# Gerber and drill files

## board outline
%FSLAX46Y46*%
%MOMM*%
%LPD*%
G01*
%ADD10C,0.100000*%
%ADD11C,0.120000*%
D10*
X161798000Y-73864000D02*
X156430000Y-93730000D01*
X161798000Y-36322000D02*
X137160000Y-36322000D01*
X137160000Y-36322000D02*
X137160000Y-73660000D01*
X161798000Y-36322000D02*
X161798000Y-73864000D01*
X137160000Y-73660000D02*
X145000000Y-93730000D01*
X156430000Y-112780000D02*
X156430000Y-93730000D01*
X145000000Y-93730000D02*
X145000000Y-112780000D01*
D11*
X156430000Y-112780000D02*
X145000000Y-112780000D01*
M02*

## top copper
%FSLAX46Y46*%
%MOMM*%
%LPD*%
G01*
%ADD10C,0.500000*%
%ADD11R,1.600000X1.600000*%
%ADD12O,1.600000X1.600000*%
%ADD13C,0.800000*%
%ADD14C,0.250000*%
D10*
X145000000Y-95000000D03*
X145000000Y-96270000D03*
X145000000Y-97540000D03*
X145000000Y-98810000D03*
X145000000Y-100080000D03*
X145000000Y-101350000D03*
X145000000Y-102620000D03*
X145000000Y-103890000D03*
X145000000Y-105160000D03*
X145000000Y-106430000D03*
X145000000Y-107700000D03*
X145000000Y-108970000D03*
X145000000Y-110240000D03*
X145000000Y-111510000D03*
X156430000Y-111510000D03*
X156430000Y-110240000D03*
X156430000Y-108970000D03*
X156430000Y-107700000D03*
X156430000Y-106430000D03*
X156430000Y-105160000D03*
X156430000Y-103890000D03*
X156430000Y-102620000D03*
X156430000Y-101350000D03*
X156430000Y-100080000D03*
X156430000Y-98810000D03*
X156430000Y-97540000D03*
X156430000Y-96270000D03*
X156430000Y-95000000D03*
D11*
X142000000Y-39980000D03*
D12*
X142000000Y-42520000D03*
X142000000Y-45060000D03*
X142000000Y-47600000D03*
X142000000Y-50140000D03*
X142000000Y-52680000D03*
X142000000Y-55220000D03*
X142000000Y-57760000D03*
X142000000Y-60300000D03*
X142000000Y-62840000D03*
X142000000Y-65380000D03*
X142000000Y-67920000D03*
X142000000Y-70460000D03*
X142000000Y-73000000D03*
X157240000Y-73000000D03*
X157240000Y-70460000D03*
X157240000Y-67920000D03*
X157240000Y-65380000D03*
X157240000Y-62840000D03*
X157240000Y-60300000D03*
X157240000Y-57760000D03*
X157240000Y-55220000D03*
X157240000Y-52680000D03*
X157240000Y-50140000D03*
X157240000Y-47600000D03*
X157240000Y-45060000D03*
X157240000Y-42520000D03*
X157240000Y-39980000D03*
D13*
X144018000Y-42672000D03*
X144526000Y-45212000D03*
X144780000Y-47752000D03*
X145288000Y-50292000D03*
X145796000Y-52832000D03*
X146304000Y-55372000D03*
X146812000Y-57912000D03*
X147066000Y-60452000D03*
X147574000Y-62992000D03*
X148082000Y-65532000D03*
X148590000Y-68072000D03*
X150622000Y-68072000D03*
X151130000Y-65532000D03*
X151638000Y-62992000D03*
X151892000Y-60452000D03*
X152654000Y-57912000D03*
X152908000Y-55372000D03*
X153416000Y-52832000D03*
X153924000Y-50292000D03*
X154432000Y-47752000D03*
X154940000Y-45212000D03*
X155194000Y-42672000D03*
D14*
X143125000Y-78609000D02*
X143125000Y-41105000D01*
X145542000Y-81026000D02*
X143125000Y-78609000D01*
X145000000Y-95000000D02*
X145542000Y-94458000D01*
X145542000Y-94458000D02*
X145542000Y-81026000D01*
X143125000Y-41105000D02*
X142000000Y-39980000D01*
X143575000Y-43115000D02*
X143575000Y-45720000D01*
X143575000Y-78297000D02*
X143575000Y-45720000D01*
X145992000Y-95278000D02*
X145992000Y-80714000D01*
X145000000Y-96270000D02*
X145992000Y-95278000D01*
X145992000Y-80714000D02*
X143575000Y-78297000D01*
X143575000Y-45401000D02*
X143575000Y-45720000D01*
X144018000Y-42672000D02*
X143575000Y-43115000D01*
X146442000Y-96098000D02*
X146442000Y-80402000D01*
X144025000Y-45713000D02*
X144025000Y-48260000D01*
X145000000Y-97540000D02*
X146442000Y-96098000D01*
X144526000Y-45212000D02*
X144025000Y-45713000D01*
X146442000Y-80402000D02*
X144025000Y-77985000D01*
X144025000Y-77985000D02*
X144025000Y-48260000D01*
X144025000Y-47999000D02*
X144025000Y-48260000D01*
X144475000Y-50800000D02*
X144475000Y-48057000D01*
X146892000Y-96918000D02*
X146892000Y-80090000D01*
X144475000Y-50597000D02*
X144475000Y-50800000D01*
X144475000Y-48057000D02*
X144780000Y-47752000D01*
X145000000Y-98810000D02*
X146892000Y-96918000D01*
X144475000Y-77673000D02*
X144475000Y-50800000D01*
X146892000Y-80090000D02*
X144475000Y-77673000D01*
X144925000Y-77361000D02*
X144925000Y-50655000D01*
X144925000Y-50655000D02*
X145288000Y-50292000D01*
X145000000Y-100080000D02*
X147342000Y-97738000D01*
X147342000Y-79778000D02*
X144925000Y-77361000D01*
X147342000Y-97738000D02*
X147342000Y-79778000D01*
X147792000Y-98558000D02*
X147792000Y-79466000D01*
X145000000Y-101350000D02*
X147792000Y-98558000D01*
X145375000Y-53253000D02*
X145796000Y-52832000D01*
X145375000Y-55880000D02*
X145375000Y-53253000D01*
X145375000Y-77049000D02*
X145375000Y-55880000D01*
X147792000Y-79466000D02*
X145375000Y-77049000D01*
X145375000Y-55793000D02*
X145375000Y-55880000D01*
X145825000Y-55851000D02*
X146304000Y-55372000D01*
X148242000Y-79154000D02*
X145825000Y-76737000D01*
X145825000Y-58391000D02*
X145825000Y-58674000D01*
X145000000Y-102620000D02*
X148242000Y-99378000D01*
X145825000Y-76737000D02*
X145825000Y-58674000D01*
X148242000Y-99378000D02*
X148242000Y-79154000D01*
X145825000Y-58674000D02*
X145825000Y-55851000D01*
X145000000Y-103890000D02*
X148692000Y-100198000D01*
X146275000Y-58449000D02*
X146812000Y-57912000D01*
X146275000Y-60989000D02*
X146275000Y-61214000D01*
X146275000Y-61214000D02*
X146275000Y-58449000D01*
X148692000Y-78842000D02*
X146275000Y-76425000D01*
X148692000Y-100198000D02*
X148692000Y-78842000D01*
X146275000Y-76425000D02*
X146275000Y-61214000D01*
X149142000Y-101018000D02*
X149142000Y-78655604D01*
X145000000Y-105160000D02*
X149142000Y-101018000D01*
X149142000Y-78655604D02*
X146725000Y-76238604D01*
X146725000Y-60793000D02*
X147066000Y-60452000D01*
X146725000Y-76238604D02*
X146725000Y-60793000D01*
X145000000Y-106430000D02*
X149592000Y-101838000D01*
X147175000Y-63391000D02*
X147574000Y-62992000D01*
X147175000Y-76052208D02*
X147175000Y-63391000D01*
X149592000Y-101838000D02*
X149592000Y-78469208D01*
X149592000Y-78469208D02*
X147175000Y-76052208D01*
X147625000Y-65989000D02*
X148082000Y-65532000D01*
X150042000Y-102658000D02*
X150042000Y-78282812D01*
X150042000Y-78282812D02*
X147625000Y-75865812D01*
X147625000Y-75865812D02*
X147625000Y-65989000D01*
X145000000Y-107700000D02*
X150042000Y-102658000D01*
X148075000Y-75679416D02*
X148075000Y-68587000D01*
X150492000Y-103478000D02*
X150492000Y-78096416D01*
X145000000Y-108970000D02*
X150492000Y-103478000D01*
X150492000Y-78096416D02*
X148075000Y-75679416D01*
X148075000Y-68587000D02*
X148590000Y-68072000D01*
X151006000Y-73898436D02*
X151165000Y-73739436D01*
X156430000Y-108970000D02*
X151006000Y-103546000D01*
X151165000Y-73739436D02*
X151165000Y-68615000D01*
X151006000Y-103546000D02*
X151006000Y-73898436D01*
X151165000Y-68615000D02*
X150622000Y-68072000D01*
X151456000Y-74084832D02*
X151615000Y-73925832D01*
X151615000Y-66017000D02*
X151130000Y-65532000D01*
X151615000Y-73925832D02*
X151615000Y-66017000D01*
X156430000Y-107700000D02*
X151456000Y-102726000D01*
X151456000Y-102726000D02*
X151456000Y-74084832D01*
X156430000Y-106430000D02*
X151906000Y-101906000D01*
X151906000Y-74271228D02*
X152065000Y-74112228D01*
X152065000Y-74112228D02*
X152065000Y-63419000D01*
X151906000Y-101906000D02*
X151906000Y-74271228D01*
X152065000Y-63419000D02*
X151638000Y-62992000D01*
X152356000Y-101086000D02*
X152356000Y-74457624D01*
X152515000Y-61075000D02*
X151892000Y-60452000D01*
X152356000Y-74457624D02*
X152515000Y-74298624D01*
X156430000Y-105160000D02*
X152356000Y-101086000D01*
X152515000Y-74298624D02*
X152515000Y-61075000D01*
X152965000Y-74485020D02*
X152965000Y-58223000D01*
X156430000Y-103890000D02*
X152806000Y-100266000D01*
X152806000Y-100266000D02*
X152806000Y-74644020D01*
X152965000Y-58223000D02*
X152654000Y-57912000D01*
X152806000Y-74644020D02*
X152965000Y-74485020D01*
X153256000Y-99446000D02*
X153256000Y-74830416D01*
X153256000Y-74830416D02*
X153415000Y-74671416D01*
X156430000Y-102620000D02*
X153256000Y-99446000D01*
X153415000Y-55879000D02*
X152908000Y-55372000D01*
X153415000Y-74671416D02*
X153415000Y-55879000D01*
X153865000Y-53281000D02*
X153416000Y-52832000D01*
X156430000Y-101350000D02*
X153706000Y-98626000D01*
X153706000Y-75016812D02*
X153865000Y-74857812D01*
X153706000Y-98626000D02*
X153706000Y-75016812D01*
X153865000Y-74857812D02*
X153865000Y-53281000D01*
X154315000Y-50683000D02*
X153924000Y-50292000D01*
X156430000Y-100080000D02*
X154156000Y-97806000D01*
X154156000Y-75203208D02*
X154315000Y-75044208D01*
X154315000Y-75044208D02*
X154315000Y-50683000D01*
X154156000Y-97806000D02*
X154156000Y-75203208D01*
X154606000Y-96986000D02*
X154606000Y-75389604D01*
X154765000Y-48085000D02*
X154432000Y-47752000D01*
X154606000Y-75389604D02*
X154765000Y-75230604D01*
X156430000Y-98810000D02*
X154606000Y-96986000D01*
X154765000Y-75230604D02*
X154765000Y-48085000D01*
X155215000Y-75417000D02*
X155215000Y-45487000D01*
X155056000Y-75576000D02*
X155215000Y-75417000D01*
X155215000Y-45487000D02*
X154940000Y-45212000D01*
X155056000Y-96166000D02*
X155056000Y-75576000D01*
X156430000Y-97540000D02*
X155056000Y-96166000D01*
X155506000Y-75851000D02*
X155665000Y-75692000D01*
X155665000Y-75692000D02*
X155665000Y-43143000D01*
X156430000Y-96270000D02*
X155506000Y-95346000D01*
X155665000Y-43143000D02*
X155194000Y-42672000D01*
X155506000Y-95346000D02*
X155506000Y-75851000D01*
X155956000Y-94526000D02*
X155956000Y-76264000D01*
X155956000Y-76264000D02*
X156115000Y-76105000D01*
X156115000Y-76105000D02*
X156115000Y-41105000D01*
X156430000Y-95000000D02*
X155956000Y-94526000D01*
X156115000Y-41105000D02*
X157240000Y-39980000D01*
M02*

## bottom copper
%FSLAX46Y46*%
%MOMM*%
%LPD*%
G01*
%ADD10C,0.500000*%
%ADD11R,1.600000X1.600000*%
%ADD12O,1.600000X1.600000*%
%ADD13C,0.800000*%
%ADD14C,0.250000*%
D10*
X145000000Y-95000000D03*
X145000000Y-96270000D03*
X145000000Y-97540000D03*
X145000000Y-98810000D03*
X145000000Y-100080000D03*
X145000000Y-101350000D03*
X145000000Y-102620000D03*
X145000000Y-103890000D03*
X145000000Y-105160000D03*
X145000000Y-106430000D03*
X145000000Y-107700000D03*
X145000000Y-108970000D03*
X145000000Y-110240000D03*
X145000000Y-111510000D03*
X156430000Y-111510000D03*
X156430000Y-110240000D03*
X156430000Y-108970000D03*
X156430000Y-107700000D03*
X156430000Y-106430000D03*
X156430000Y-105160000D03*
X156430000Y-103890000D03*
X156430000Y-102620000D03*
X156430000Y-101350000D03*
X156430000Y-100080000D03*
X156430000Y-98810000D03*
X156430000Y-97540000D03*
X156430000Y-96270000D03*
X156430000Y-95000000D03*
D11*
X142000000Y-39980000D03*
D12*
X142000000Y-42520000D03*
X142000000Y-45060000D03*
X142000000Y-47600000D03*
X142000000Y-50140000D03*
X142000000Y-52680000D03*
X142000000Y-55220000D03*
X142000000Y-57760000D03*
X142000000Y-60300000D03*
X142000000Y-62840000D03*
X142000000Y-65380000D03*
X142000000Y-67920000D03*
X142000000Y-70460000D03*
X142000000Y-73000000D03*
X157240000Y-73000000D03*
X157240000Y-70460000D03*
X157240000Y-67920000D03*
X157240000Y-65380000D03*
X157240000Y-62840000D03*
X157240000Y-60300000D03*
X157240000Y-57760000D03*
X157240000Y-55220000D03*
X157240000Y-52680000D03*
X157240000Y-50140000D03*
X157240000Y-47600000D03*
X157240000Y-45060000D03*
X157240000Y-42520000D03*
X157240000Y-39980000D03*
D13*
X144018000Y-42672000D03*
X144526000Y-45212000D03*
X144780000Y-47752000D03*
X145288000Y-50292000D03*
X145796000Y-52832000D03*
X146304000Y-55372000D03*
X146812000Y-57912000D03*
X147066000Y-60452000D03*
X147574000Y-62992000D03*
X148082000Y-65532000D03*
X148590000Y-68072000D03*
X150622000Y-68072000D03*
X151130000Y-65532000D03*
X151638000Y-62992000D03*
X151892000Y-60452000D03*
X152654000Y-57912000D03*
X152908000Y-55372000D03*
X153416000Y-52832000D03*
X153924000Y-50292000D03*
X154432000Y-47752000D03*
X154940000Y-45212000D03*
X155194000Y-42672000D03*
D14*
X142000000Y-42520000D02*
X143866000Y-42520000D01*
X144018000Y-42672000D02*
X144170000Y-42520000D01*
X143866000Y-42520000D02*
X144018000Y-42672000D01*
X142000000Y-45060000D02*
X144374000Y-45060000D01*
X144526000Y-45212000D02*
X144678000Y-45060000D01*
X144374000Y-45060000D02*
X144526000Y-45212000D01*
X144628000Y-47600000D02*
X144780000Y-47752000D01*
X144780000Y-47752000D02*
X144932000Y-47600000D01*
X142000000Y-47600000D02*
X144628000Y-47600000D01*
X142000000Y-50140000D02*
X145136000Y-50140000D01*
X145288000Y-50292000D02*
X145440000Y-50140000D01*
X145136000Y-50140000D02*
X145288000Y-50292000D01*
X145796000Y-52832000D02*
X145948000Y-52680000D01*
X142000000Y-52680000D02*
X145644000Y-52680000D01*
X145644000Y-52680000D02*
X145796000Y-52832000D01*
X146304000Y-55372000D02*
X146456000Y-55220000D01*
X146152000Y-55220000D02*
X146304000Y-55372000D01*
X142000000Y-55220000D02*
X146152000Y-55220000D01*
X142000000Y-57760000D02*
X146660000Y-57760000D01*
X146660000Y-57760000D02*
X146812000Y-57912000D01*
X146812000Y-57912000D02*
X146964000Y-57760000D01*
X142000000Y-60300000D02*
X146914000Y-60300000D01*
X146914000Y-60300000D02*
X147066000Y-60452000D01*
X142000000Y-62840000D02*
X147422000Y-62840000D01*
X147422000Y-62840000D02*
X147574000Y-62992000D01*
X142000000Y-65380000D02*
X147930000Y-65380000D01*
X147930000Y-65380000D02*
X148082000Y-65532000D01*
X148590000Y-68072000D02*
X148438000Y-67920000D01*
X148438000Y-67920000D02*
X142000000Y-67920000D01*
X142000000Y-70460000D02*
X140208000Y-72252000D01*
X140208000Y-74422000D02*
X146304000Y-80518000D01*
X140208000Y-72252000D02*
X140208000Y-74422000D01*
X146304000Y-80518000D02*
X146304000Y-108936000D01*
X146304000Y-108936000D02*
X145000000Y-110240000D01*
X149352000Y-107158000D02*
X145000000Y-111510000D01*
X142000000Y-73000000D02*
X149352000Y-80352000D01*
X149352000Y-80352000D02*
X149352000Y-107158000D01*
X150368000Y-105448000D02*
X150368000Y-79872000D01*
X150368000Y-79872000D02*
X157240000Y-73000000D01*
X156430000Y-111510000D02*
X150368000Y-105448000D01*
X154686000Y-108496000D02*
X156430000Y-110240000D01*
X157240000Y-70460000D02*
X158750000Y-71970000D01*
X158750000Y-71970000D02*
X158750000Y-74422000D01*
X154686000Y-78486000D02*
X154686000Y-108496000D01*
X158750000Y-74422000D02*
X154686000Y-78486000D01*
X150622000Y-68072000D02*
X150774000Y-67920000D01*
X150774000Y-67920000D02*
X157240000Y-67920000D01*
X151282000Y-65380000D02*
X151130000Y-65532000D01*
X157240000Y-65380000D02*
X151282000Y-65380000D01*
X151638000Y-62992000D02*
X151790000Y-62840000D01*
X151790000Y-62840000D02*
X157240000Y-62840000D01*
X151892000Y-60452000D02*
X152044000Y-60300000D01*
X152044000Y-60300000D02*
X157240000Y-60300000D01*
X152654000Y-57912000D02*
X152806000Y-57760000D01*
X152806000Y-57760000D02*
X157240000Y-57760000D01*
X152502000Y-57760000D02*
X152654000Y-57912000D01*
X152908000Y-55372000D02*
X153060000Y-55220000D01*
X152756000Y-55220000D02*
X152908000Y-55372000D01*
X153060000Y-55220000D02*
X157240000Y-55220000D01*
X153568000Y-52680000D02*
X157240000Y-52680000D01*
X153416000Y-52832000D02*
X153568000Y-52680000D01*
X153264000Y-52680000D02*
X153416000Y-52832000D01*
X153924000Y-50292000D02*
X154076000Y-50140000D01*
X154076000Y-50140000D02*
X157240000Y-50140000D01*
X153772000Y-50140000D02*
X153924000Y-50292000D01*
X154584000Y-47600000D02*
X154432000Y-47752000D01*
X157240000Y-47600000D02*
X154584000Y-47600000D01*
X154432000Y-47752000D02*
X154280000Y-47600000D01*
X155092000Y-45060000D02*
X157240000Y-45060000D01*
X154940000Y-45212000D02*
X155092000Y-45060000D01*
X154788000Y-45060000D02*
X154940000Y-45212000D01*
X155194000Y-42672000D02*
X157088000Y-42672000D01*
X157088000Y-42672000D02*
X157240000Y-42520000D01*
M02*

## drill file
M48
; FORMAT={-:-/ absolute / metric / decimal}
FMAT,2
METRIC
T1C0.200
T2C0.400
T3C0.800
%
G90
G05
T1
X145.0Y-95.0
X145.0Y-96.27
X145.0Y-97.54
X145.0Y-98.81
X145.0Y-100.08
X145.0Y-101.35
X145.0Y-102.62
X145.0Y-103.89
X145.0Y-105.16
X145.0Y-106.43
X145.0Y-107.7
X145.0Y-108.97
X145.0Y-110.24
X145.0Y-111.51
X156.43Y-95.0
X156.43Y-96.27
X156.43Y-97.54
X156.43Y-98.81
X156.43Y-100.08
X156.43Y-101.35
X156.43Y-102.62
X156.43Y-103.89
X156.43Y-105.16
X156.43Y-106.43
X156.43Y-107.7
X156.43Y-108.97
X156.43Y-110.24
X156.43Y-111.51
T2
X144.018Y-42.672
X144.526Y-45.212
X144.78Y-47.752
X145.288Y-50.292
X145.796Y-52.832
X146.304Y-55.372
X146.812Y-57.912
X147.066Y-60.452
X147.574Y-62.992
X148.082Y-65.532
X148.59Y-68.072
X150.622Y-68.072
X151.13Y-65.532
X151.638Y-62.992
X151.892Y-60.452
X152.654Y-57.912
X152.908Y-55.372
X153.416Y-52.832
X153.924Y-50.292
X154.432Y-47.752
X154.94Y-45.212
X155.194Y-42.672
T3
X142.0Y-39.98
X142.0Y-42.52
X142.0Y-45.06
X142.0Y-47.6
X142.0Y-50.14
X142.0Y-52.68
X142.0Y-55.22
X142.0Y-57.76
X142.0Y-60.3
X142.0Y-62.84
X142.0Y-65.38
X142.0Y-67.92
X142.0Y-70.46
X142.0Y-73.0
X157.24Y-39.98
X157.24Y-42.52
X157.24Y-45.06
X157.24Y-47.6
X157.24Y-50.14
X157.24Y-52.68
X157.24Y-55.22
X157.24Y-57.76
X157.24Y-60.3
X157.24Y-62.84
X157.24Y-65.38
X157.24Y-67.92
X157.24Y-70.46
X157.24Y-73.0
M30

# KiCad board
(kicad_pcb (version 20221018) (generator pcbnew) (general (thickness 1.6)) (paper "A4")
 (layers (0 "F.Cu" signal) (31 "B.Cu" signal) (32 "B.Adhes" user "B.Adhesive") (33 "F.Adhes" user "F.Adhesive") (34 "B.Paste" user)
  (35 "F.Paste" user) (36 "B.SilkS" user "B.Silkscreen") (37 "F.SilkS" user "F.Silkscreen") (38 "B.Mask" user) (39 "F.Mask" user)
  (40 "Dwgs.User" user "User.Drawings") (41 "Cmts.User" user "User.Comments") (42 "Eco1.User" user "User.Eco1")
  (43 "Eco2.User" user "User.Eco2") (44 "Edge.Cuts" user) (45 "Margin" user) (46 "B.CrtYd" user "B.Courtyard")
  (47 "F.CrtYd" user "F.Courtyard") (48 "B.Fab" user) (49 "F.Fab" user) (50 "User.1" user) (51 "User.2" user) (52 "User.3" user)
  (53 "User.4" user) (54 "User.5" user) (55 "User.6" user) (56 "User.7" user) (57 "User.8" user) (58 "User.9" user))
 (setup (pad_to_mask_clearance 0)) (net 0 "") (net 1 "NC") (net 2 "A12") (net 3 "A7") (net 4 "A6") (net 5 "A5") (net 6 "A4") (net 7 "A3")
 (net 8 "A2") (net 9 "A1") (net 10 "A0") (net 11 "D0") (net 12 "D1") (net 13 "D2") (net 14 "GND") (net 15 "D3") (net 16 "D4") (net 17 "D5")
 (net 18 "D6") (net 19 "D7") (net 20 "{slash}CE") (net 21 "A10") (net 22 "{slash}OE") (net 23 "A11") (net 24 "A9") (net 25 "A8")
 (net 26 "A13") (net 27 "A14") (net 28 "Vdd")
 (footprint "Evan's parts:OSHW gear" (layer "F.Cu") (at 149.86 45.212)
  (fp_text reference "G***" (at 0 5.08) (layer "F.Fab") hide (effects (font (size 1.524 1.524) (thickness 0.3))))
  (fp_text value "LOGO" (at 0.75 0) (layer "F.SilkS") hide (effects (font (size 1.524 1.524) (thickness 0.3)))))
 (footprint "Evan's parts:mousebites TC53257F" (layer "F.Cu") (at 145 95)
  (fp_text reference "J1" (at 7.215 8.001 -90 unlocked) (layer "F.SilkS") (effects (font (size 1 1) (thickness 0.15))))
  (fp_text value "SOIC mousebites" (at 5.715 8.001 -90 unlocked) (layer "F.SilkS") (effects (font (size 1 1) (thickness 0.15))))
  (fp_line (start 11.43 17.78) (end 0 17.78) (stroke (width 0.12) (type default)) (layer "Edge.Cuts"))
  (pad "1" thru_hole circle (at 0 0) (size 0.5 0.5) (drill 0.2) (layers "*.Cu" "*.Mask") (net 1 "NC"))
  (pad "2" thru_hole circle (at 0 1.27) (size 0.5 0.5) (drill 0.2) (layers "*.Cu" "*.Mask") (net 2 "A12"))
  (pad "3" thru_hole circle (at 0 2.54) (size 0.5 0.5) (drill 0.2) (layers "*.Cu" "*.Mask") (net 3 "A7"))
  (pad "4" thru_hole circle (at 0 3.81) (size 0.5 0.5) (drill 0.2) (layers "*.Cu" "*.Mask") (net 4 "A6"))
  (pad "5" thru_hole circle (at 0 5.08) (size 0.5 0.5) (drill 0.2) (layers "*.Cu" "*.Mask") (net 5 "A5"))
  (pad "6" thru_hole circle (at 0 6.35) (size 0.5 0.5) (drill 0.2) (layers "*.Cu" "*.Mask") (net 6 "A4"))
  (pad "7" thru_hole circle (at 0 7.62) (size 0.5 0.5) (drill 0.2) (layers "*.Cu" "*.Mask") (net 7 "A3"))
  (pad "8" thru_hole circle (at 0 8.89) (size 0.5 0.5) (drill 0.2) (layers "*.Cu" "*.Mask") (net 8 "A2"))
  (pad "9" thru_hole circle (at 0 10.16) (size 0.5 0.5) (drill 0.2) (layers "*.Cu" "*.Mask") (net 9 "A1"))
  (pad "10" thru_hole circle (at 0 11.43) (size 0.5 0.5) (drill 0.2) (layers "*.Cu" "*.Mask") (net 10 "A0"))
  (pad "11" thru_hole circle (at 0 12.7) (size 0.5 0.5) (drill 0.2) (layers "*.Cu" "*.Mask") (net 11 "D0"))
  (pad "12" thru_hole circle (at 0 13.97) (size 0.5 0.5) (drill 0.2) (layers "*.Cu" "*.Mask") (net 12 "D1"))
  (pad "13" thru_hole circle (at 0 15.24) (size 0.5 0.5) (drill 0.2) (layers "*.Cu" "*.Mask") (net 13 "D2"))
  (pad "14" thru_hole circle (at 0 16.51) (size 0.5 0.5) (drill 0.2) (layers "*.Cu" "*.Mask") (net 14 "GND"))
  (pad "15" thru_hole circle (at 11.43 16.51) (size 0.5 0.5) (drill 0.2) (layers "*.Cu" "*.Mask") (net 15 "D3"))
  (pad "16" thru_hole circle (at 11.43 15.24) (size 0.5 0.5) (drill 0.2) (layers "*.Cu" "*.Mask") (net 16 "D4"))
  (pad "17" thru_hole circle (at 11.43 13.97) (size 0.5 0.5) (drill 0.2) (layers "*.Cu" "*.Mask") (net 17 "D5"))
  (pad "18" thru_hole circle (at 11.43 12.7) (size 0.5 0.5) (drill 0.2) (layers "*.Cu" "*.Mask") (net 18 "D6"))
  (pad "19" thru_hole circle (at 11.43 11.43) (size 0.5 0.5) (drill 0.2) (layers "*.Cu" "*.Mask") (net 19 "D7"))
  (pad "20" thru_hole circle (at 11.43 10.16) (size 0.5 0.5) (drill 0.2) (layers "*.Cu" "*.Mask") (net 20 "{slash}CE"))
  (pad "21" thru_hole circle (at 11.43 8.89) (size 0.5 0.5) (drill 0.2) (layers "*.Cu" "*.Mask") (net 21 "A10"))
  (pad "22" thru_hole circle (at 11.43 7.62) (size 0.5 0.5) (drill 0.2) (layers "*.Cu" "*.Mask") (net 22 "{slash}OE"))
  (pad "23" thru_hole circle (at 11.43 6.35) (size 0.5 0.5) (drill 0.2) (layers "*.Cu" "*.Mask") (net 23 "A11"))
  (pad "24" thru_hole circle (at 11.43 5.08) (size 0.5 0.5) (drill 0.2) (layers "*.Cu" "*.Mask") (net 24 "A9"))
  (pad "25" thru_hole circle (at 11.43 3.81) (size 0.5 0.5) (drill 0.2) (layers "*.Cu" "*.Mask") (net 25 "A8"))
  (pad "26" thru_hole circle (at 11.43 2.54) (size 0.5 0.5) (drill 0.2) (layers "*.Cu" "*.Mask") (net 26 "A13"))
  (pad "27" thru_hole circle (at 11.43 1.27) (size 0.5 0.5) (drill 0.2) (layers "*.Cu" "*.Mask") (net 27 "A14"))
  (pad "28" thru_hole circle (at 11.43 0) (size 0.5 0.5) (drill 0.2) (layers "*.Cu" "*.Mask") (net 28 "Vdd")))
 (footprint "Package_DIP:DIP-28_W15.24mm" (layer "F.Cu") (at 142 39.98)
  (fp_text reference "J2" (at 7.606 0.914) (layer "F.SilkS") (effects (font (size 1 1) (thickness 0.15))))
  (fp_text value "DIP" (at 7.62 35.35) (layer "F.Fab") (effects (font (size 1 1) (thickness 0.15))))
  (pad "1" thru_hole rect (at 0 0) (size 1.6 1.6) (drill 0.8) (layers "*.Cu" "*.Mask") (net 1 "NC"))
  (pad "2" thru_hole oval (at 0 2.54) (size 1.6 1.6) (drill 0.8) (layers "*.Cu" "*.Mask") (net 2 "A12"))
  (pad "3" thru_hole oval (at 0 5.08) (size 1.6 1.6) (drill 0.8) (layers "*.Cu" "*.Mask") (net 3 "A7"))
  (pad "4" thru_hole oval (at 0 7.62) (size 1.6 1.6) (drill 0.8) (layers "*.Cu" "*.Mask") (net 4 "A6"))
  (pad "5" thru_hole oval (at 0 10.16) (size 1.6 1.6) (drill 0.8) (layers "*.Cu" "*.Mask") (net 5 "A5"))
  (pad "6" thru_hole oval (at 0 12.7) (size 1.6 1.6) (drill 0.8) (layers "*.Cu" "*.Mask") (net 6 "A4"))
  (pad "7" thru_hole oval (at 0 15.24) (size 1.6 1.6) (drill 0.8) (layers "*.Cu" "*.Mask") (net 7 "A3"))
  (pad "8" thru_hole oval (at 0 17.78) (size 1.6 1.6) (drill 0.8) (layers "*.Cu" "*.Mask") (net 8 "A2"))
  (pad "9" thru_hole oval (at 0 20.32) (size 1.6 1.6) (drill 0.8) (layers "*.Cu" "*.Mask") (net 9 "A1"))
  (pad "10" thru_hole oval (at 0 22.86) (size 1.6 1.6) (drill 0.8) (layers "*.Cu" "*.Mask") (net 10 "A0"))
  (pad "11" thru_hole oval (at 0 25.4) (size 1.6 1.6) (drill 0.8) (layers "*.Cu" "*.Mask") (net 11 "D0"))
  (pad "12" thru_hole oval (at 0 27.94) (size 1.6 1.6) (drill 0.8) (layers "*.Cu" "*.Mask") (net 12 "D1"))
  (pad "13" thru_hole oval (at 0 30.48) (size 1.6 1.6) (drill 0.8) (layers "*.Cu" "*.Mask") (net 13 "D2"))
  (pad "14" thru_hole oval (at 0 33.02) (size 1.6 1.6) (drill 0.8) (layers "*.Cu" "*.Mask") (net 14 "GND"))
  (pad "15" thru_hole oval (at 15.24 33.02) (size 1.6 1.6) (drill 0.8) (layers "*.Cu" "*.Mask") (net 15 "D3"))
  (pad "16" thru_hole oval (at 15.24 30.48) (size 1.6 1.6) (drill 0.8) (layers "*.Cu" "*.Mask") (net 16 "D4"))
  (pad "17" thru_hole oval (at 15.24 27.94) (size 1.6 1.6) (drill 0.8) (layers "*.Cu" "*.Mask") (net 17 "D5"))
  (pad "18" thru_hole oval (at 15.24 25.4) (size 1.6 1.6) (drill 0.8) (layers "*.Cu" "*.Mask") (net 18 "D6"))
  (pad "19" thru_hole oval (at 15.24 22.86) (size 1.6 1.6) (drill 0.8) (layers "*.Cu" "*.Mask") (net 19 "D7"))
  (pad "20" thru_hole oval (at 15.24 20.32) (size 1.6 1.6) (drill 0.8) (layers "*.Cu" "*.Mask") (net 20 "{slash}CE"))
  (pad "21" thru_hole oval (at 15.24 17.78) (size 1.6 1.6) (drill 0.8) (layers "*.Cu" "*.Mask") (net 21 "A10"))
  (pad "22" thru_hole oval (at 15.24 15.24) (size 1.6 1.6) (drill 0.8) (layers "*.Cu" "*.Mask") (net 22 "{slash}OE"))
  (pad "23" thru_hole oval (at 15.24 12.7) (size 1.6 1.6) (drill 0.8) (layers "*.Cu" "*.Mask") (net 23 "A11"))
  (pad "24" thru_hole oval (at 15.24 10.16) (size 1.6 1.6) (drill 0.8) (layers "*.Cu" "*.Mask") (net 24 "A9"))
  (pad "25" thru_hole oval (at 15.24 7.62) (size 1.6 1.6) (drill 0.8) (layers "*.Cu" "*.Mask") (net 25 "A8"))
  (pad "26" thru_hole oval (at 15.24 5.08) (size 1.6 1.6) (drill 0.8) (layers "*.Cu" "*.Mask") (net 26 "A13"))
  (pad "27" thru_hole oval (at 15.24 2.54) (size 1.6 1.6) (drill 0.8) (layers "*.Cu" "*.Mask") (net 27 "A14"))
  (pad "28" thru_hole oval (at 15.24 0) (size 1.6 1.6) (drill 0.8) (layers "*.Cu" "*.Mask") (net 28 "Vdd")))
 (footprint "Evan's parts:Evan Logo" (layer "B.Cu") (at 149.86 41.402 -90)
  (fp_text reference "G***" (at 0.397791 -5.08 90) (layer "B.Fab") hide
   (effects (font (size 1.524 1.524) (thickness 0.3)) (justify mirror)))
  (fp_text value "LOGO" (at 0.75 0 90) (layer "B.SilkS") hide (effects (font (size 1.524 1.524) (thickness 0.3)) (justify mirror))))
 (gr_line (start 161.798 73.864) (end 156.43 93.73) (stroke (width 0.1) (type default)) (layer "Edge.Cuts"))
 (gr_line (start 161.798 36.322) (end 137.16 36.322) (stroke (width 0.1) (type default)) (layer "Edge.Cuts"))
 (gr_line (start 137.16 36.322) (end 137.16 73.66) (stroke (width 0.1) (type default)) (layer "Edge.Cuts"))
 (gr_line (start 161.798 36.322) (end 161.798 73.864) (stroke (width 0.1) (type default)) (layer "Edge.Cuts"))
 (gr_line (start 137.16 73.66) (end 145 93.73) (stroke (width 0.1) (type default)) (layer "Edge.Cuts"))
 (gr_line (start 156.43 112.78) (end 156.43 93.73) (stroke (width 0.1) (type default)) (layer "Edge.Cuts"))
 (gr_line (start 145 93.73) (end 145 112.78) (stroke (width 0.1) (type default)) (layer "Edge.Cuts"))
 (segment (start 143.125 78.609) (end 143.125 41.105) (width 0.25) (layer "F.Cu") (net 1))
 (segment (start 145.542 81.026) (end 143.125 78.609) (width 0.25) (layer "F.Cu") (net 1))
 (segment (start 145 95) (end 145.542 94.458) (width 0.25) (layer "F.Cu") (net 1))
 (segment (start 145.542 94.458) (end 145.542 81.026) (width 0.25) (layer "F.Cu") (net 1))
 (segment (start 143.125 41.105) (end 142 39.98) (width 0.25) (layer "F.Cu") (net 1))
 (segment (start 143.575 43.115) (end 143.575 45.72) (width 0.25) (layer "F.Cu") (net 2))
 (segment (start 143.575 78.297) (end 143.575 45.72) (width 0.25) (layer "F.Cu") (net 2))
 (segment (start 145.992 95.278) (end 145.992 80.714) (width 0.25) (layer "F.Cu") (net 2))
 (segment (start 145 96.27) (end 145.992 95.278) (width 0.25) (layer "F.Cu") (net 2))
 (segment (start 145.992 80.714) (end 143.575 78.297) (width 0.25) (layer "F.Cu") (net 2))
 (segment (start 143.575 45.401) (end 143.575 45.72) (width 0.25) (layer "F.Cu") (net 2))
 (segment (start 144.018 42.672) (end 143.575 43.115) (width 0.25) (layer "F.Cu") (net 2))
 (via (at 144.018 42.672) (size 0.8) (drill 0.4) (layers "F.Cu" "B.Cu") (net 2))
 (segment (start 142 42.52) (end 143.866 42.52) (width 0.25) (layer "B.Cu") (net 2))
 (segment (start 144.018 42.672) (end 144.17 42.52) (width 0.25) (layer "B.Cu") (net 2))
 (segment (start 143.866 42.52) (end 144.018 42.672) (width 0.25) (layer "B.Cu") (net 2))
 (segment (start 146.442 96.098) (end 146.442 80.402) (width 0.25) (layer "F.Cu") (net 3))
 (segment (start 144.025 45.713) (end 144.025 48.26) (width 0.25) (layer "F.Cu") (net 3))
 (segment (start 145 97.54) (end 146.442 96.098) (width 0.25) (layer "F.Cu") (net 3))
 (segment (start 144.526 45.212) (end 144.025 45.713) (width 0.25) (layer "F.Cu") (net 3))
 (segment (start 146.442 80.402) (end 144.025 77.985) (width 0.25) (layer "F.Cu") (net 3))
 (segment (start 144.025 77.985) (end 144.025 48.26) (width 0.25) (layer "F.Cu") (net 3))
 (segment (start 144.025 47.999) (end 144.025 48.26) (width 0.25) (layer "F.Cu") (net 3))
 (via (at 144.526 45.212) (size 0.8) (drill 0.4) (layers "F.Cu" "B.Cu") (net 3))
 (segment (start 142 45.06) (end 144.374 45.06) (width 0.25) (layer "B.Cu") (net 3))
 (segment (start 144.526 45.212) (end 144.678 45.06) (width 0.25) (layer "B.Cu") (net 3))
 (segment (start 144.374 45.06) (end 144.526 45.212) (width 0.25) (layer "B.Cu") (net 3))
 (segment (start 144.475 50.8) (end 144.475 48.057) (width 0.25) (layer "F.Cu") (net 4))
 (segment (start 146.892 96.918) (end 146.892 80.09) (width 0.25) (layer "F.Cu") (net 4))
 (segment (start 144.475 50.597) (end 144.475 50.8) (width 0.25) (layer "F.Cu") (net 4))
 (segment (start 144.475 48.057) (end 144.78 47.752) (width 0.25) (layer "F.Cu") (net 4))
 (segment (start 145 98.81) (end 146.892 96.918) (width 0.25) (layer "F.Cu") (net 4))
 (segment (start 144.475 77.673) (end 144.475 50.8) (width 0.25) (layer "F.Cu") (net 4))
 (segment (start 146.892 80.09) (end 144.475 77.673) (width 0.25) (layer "F.Cu") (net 4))
 (via (at 144.78 47.752) (size 0.8) (drill 0.4) (layers "F.Cu" "B.Cu") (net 4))
 (segment (start 144.628 47.6) (end 144.78 47.752) (width 0.25) (layer "B.Cu") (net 4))
 (segment (start 144.78 47.752) (end 144.932 47.6) (width 0.25) (layer "B.Cu") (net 4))
 (segment (start 142 47.6) (end 144.628 47.6) (width 0.25) (layer "B.Cu") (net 4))
 (segment (start 144.925 77.361) (end 144.925 50.655) (width 0.25) (layer "F.Cu") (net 5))
 (segment (start 144.925 50.655) (end 145.288 50.292) (width 0.25) (layer "F.Cu") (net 5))
 (segment (start 145 100.08) (end 147.342 97.738) (width 0.25) (layer "F.Cu") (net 5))
 (segment (start 147.342 79.778) (end 144.925 77.361) (width 0.25) (layer "F.Cu") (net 5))
 (segment (start 147.342 97.738) (end 147.342 79.778) (width 0.25) (layer "F.Cu") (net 5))
 (via (at 145.288 50.292) (size 0.8) (drill 0.4) (layers "F.Cu" "B.Cu") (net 5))
 (segment (start 142 50.14) (end 145.136 50.14) (width 0.25) (layer "B.Cu") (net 5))
 (segment (start 145.288 50.292) (end 145.44 50.14) (width 0.25) (layer "B.Cu") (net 5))
 (segment (start 145.136 50.14) (end 145.288 50.292) (width 0.25) (layer "B.Cu") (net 5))
 (segment (start 147.792 98.558) (end 147.792 79.466) (width 0.25) (layer "F.Cu") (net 6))
 (segment (start 145 101.35) (end 147.792 98.558) (width 0.25) (layer "F.Cu") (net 6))
 (segment (start 145.375 53.253) (end 145.796 52.832) (width 0.25) (layer "F.Cu") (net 6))
 (segment (start 145.375 55.88) (end 145.375 53.253) (width 0.25) (layer "F.Cu") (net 6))
 (segment (start 145.375 77.049) (end 145.375 55.88) (width 0.25) (layer "F.Cu") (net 6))
 (segment (start 147.792 79.466) (end 145.375 77.049) (width 0.25) (layer "F.Cu") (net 6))
 (segment (start 145.375 55.793) (end 145.375 55.88) (width 0.25) (layer "F.Cu") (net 6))
 (via (at 145.796 52.832) (size 0.8) (drill 0.4) (layers "F.Cu" "B.Cu") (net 6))
 (segment (start 145.796 52.832) (end 145.948 52.68) (width 0.25) (layer "B.Cu") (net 6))
 (segment (start 142 52.68) (end 145.644 52.68) (width 0.25) (layer "B.Cu") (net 6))
 (segment (start 145.644 52.68) (end 145.796 52.832) (width 0.25) (layer "B.Cu") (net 6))
 (segment (start 145.825 55.851) (end 146.304 55.372) (width 0.25) (layer "F.Cu") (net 7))
 (segment (start 148.242 79.154) (end 145.825 76.737) (width 0.25) (layer "F.Cu") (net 7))
 (segment (start 145.825 58.391) (end 145.825 58.674) (width 0.25) (layer "F.Cu") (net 7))
 (segment (start 145 102.62) (end 148.242 99.378) (width 0.25) (layer "F.Cu") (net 7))
 (segment (start 145.825 76.737) (end 145.825 58.674) (width 0.25) (layer "F.Cu") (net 7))
 (segment (start 148.242 99.378) (end 148.242 79.154) (width 0.25) (layer "F.Cu") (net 7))
 (segment (start 145.825 58.674) (end 145.825 55.851) (width 0.25) (layer "F.Cu") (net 7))
 (via (at 146.304 55.372) (size 0.8) (drill 0.4) (layers "F.Cu" "B.Cu") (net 7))
 (segment (start 146.304 55.372) (end 146.456 55.22) (width 0.25) (layer "B.Cu") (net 7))
 (segment (start 146.152 55.22) (end 146.304 55.372) (width 0.25) (layer "B.Cu") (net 7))
 (segment (start 142 55.22) (end 146.152 55.22) (width 0.25) (layer "B.Cu") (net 7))
 (segment (start 145 103.89) (end 148.692 100.198) (width 0.25) (layer "F.Cu") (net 8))
 (segment (start 146.275 58.449) (end 146.812 57.912) (width 0.25) (layer "F.Cu") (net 8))
 (segment (start 146.275 60.989) (end 146.275 61.214) (width 0.25) (layer "F.Cu") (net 8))
 (segment (start 146.275 61.214) (end 146.275 58.449) (width 0.25) (layer "F.Cu") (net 8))
 (segment (start 148.692 78.842) (end 146.275 76.425) (width 0.25) (layer "F.Cu") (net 8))
 (segment (start 148.692 100.198) (end 148.692 78.842) (width 0.25) (layer "F.Cu") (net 8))
 (segment (start 146.275 76.425) (end 146.275 61.214) (width 0.25) (layer "F.Cu") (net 8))
 (via (at 146.812 57.912) (size 0.8) (drill 0.4) (layers "F.Cu" "B.Cu") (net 8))
 (segment (start 142 57.76) (end 146.66 57.76) (width 0.25) (layer "B.Cu") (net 8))
 (segment (start 146.66 57.76) (end 146.812 57.912) (width 0.25) (layer "B.Cu") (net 8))
 (segment (start 146.812 57.912) (end 146.964 57.76) (width 0.25) (layer "B.Cu") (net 8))
 (segment (start 149.142 101.018) (end 149.142 78.655604) (width 0.25) (layer "F.Cu") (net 9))
 (segment (start 145 105.16) (end 149.142 101.018) (width 0.25) (layer "F.Cu") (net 9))
 (segment (start 149.142 78.655604) (end 146.725 76.238604) (width 0.25) (layer "F.Cu") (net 9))
 (segment (start 146.725 60.793) (end 147.066 60.452) (width 0.25) (layer "F.Cu") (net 9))
 (segment (start 146.725 76.238604) (end 146.725 60.793) (width 0.25) (layer "F.Cu") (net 9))
 (via (at 147.066 60.452) (size 0.8) (drill 0.4) (layers "F.Cu" "B.Cu") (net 9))
 (segment (start 142 60.3) (end 146.914 60.3) (width 0.25) (layer "B.Cu") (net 9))
 (segment (start 146.914 60.3) (end 147.066 60.452) (width 0.25) (layer "B.Cu") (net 9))
 (segment (start 145 106.43) (end 149.592 101.838) (width 0.25) (layer "F.Cu") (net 10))
 (segment (start 147.175 63.391) (end 147.574 62.992) (width 0.25) (layer "F.Cu") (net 10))
 (segment (start 147.175 76.052208) (end 147.175 63.391) (width 0.25) (layer "F.Cu") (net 10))
 (segment (start 149.592 101.838) (end 149.592 78.469208) (width 0.25) (layer "F.Cu") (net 10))
 (segment (start 149.592 78.469208) (end 147.175 76.052208) (width 0.25) (layer "F.Cu") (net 10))
 (via (at 147.574 62.992) (size 0.8) (drill 0.4) (layers "F.Cu" "B.Cu") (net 10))
 (segment (start 142 62.84) (end 147.422 62.84) (width 0.25) (layer "B.Cu") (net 10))
 (segment (start 147.422 62.84) (end 147.574 62.992) (width 0.25) (layer "B.Cu") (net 10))
 (segment (start 147.625 65.989) (end 148.082 65.532) (width 0.25) (layer "F.Cu") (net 11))
 (segment (start 150.042 102.658) (end 150.042 78.282812) (width 0.25) (layer "F.Cu") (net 11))
 (segment (start 150.042 78.282812) (end 147.625 75.865812) (width 0.25) (layer "F.Cu") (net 11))
 (segment (start 147.625 75.865812) (end 147.625 65.989) (width 0.25) (layer "F.Cu") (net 11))
 (segment (start 145 107.7) (end 150.042 102.658) (width 0.25) (layer "F.Cu") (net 11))
 (via (at 148.082 65.532) (size 0.8) (drill 0.4) (layers "F.Cu" "B.Cu") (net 11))
 (segment (start 142 65.38) (end 147.93 65.38) (width 0.25) (layer "B.Cu") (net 11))
 (segment (start 147.93 65.38) (end 148.082 65.532) (width 0.25) (layer "B.Cu") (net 11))
 (segment (start 148.075 75.679416) (end 148.075 68.587) (width 0.25) (layer "F.Cu") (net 12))
 (segment (start 150.492 103.478) (end 150.492 78.096416) (width 0.25) (layer "F.Cu") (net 12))
 (segment (start 145 108.97) (end 150.492 103.478) (width 0.25) (layer "F.Cu") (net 12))
 (segment (start 150.492 78.096416) (end 148.075 75.679416) (width 0.25) (layer "F.Cu") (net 12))
 (segment (start 148.075 68.587) (end 148.59 68.072) (width 0.25) (layer "F.Cu") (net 12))
 (via (at 148.59 68.072) (size 0.8) (drill 0.4) (layers "F.Cu" "B.Cu") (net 12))
 (segment (start 148.59 68.072) (end 148.438 67.92) (width 0.25) (layer "B.Cu") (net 12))
 (segment (start 148.438 67.92) (end 142 67.92) (width 0.25) (layer "B.Cu") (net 12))
 (segment (start 142 70.46) (end 140.208 72.252) (width 0.25) (layer "B.Cu") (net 13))
 (segment (start 140.208 74.422) (end 146.304 80.518) (width 0.25) (layer "B.Cu") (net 13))
 (segment (start 140.208 72.252) (end 140.208 74.422) (width 0.25) (layer "B.Cu") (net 13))
 (segment (start 146.304 80.518) (end 146.304 108.936) (width 0.25) (layer "B.Cu") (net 13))
 (segment (start 146.304 108.936) (end 145 110.24) (width 0.25) (layer "B.Cu") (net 13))
 (segment (start 149.352 107.158) (end 145 111.51) (width 0.25) (layer "B.Cu") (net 14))
 (segment (start 142 73) (end 149.352 80.352) (width 0.25) (layer "B.Cu") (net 14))
 (segment (start 149.352 80.352) (end 149.352 107.158) (width 0.25) (layer "B.Cu") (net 14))
 (segment (start 150.368 105.448) (end 150.368 79.872) (width 0.25) (layer "B.Cu") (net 15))
 (segment (start 150.368 79.872) (end 157.24 73) (width 0.25) (layer "B.Cu") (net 15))
 (segment (start 156.43 111.51) (end 150.368 105.448) (width 0.25) (layer "B.Cu") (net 15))
 (segment (start 154.686 108.496) (end 156.43 110.24) (width 0.25) (layer "B.Cu") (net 16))
 (segment (start 157.24 70.46) (end 158.75 71.97) (width 0.25) (layer "B.Cu") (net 16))
 (segment (start 158.75 71.97) (end 158.75 74.422) (width 0.25) (layer "B.Cu") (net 16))
 (segment (start 154.686 78.486) (end 154.686 108.496) (width 0.25) (layer "B.Cu") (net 16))
 (segment (start 158.75 74.422) (end 154.686 78.486) (width 0.25) (layer "B.Cu") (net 16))
 (segment (start 151.006 73.898436) (end 151.165 73.739436) (width 0.25) (layer "F.Cu") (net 17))
 (segment (start 156.43 108.97) (end 151.006 103.546) (width 0.25) (layer "F.Cu") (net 17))
 (segment (start 151.165 73.739436) (end 151.165 68.615) (width 0.25) (layer "F.Cu") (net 17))
 (segment (start 151.006 103.546) (end 151.006 73.898436) (width 0.25) (layer "F.Cu") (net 17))
 (segment (start 151.165 68.615) (end 150.622 68.072) (width 0.25) (layer "F.Cu") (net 17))
 (via (at 150.622 68.072) (size 0.8) (drill 0.4) (layers "F.Cu" "B.Cu") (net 17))
 (segment (start 150.622 68.072) (end 150.774 67.92) (width 0.25) (layer "B.Cu") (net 17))
 (segment (start 150.774 67.92) (end 157.24 67.92) (width 0.25) (layer "B.Cu") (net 17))
 (segment (start 151.456 74.084832) (end 151.615 73.925832) (width 0.25) (layer "F.Cu") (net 18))
 (segment (start 151.615 66.017) (end 151.13 65.532) (width 0.25) (layer "F.Cu") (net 18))
 (segment (start 151.615 73.925832) (end 151.615 66.017) (width 0.25) (layer "F.Cu") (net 18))
 (segment (start 156.43 107.7) (end 151.456 102.726) (width 0.25) (layer "F.Cu") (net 18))
 (segment (start 151.456 102.726) (end 151.456 74.084832) (width 0.25) (layer "F.Cu") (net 18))
 (via (at 151.13 65.532) (size 0.8) (drill 0.4) (layers "F.Cu" "B.Cu") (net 18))
 (segment (start 151.282 65.38) (end 151.13 65.532) (width 0.25) (layer "B.Cu") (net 18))
 (segment (start 157.24 65.38) (end 151.282 65.38) (width 0.25) (layer "B.Cu") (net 18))
 (segment (start 156.43 106.43) (end 151.906 101.906) (width 0.25) (layer "F.Cu") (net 19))
 (segment (start 151.906 74.271228) (end 152.065 74.112228) (width 0.25) (layer "F.Cu") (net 19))
 (segment (start 152.065 74.112228) (end 152.065 63.419) (width 0.25) (layer "F.Cu") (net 19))
 (segment (start 151.906 101.906) (end 151.906 74.271228) (width 0.25) (layer "F.Cu") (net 19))
 (segment (start 152.065 63.419) (end 151.638 62.992) (width 0.25) (layer "F.Cu") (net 19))
 (via (at 151.638 62.992) (size 0.8) (drill 0.4) (layers "F.Cu" "B.Cu") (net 19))
 (segment (start 151.638 62.992) (end 151.79 62.84) (width 0.25) (layer "B.Cu") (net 19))
 (segment (start 151.79 62.84) (end 157.24 62.84) (width 0.25) (layer "B.Cu") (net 19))
 (segment (start 152.356 101.086) (end 152.356 74.457624) (width 0.25) (layer "F.Cu") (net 20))
 (segment (start 152.515 61.075) (end 151.892 60.452) (width 0.25) (layer "F.Cu") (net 20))
 (segment (start 152.356 74.457624) (end 152.515 74.298624) (width 0.25) (layer "F.Cu") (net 20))
 (segment (start 156.43 105.16) (end 152.356 101.086) (width 0.25) (layer "F.Cu") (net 20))
 (segment (start 152.515 74.298624) (end 152.515 61.075) (width 0.25) (layer "F.Cu") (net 20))
 (via (at 151.892 60.452) (size 0.8) (drill 0.4) (layers "F.Cu" "B.Cu") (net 20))
 (segment (start 151.892 60.452) (end 152.044 60.3) (width 0.25) (layer "B.Cu") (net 20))
 (segment (start 152.044 60.3) (end 157.24 60.3) (width 0.25) (layer "B.Cu") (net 20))
 (segment (start 152.965 74.48502) (end 152.965 58.223) (width 0.25) (layer "F.Cu") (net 21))
 (segment (start 156.43 103.89) (end 152.806 100.266) (width 0.25) (layer "F.Cu") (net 21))
 (segment (start 152.806 100.266) (end 152.806 74.64402) (width 0.25) (layer "F.Cu") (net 21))
 (segment (start 152.965 58.223) (end 152.654 57.912) (width 0.25) (layer "F.Cu") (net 21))
 (segment (start 152.806 74.64402) (end 152.965 74.48502) (width 0.25) (layer "F.Cu") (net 21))
 (via (at 152.654 57.912) (size 0.8) (drill 0.4) (layers "F.Cu" "B.Cu") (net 21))
 (segment (start 152.654 57.912) (end 152.806 57.76) (width 0.25) (layer "B.Cu") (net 21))
 (segment (start 152.806 57.76) (end 157.24 57.76) (width 0.25) (layer "B.Cu") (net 21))
 (segment (start 152.502 57.76) (end 152.654 57.912) (width 0.25) (layer "B.Cu") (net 21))
 (segment (start 153.256 99.446) (end 153.256 74.830416) (width 0.25) (layer "F.Cu") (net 22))
 (segment (start 153.256 74.830416) (end 153.415 74.671416) (width 0.25) (layer "F.Cu") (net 22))
 (segment (start 156.43 102.62) (end 153.256 99.446) (width 0.25) (layer "F.Cu") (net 22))
 (segment (start 153.415 55.879) (end 152.908 55.372) (width 0.25) (layer "F.Cu") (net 22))
 (segment (start 153.415 74.671416) (end 153.415 55.879) (width 0.25) (layer "F.Cu") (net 22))
 (via (at 152.908 55.372) (size 0.8) (drill 0.4) (layers "F.Cu" "B.Cu") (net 22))
 (segment (start 152.908 55.372) (end 153.06 55.22) (width 0.25) (layer "B.Cu") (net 22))
 (segment (start 152.756 55.22) (end 152.908 55.372) (width 0.25) (layer "B.Cu") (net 22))
 (segment (start 153.06 55.22) (end 157.24 55.22) (width 0.25) (layer "B.Cu") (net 22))
 (segment (start 153.865 53.281) (end 153.416 52.832) (width 0.25) (layer "F.Cu") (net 23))
 (segment (start 156.43 101.35) (end 153.706 98.626) (width 0.25) (layer "F.Cu") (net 23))
 (segment (start 153.706 75.016812) (end 153.865 74.857812) (width 0.25) (layer "F.Cu") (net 23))
 (segment (start 153.706 98.626) (end 153.706 75.016812) (width 0.25) (layer "F.Cu") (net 23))
 (segment (start 153.865 74.857812) (end 153.865 53.281) (width 0.25) (layer "F.Cu") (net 23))
 (via (at 153.416 52.832) (size 0.8) (drill 0.4) (layers "F.Cu" "B.Cu") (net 23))
 (segment (start 153.568 52.68) (end 157.24 52.68) (width 0.25) (layer "B.Cu") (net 23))
 (segment (start 153.416 52.832) (end 153.568 52.68) (width 0.25) (layer "B.Cu") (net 23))
 (segment (start 153.264 52.68) (end 153.416 52.832) (width 0.25) (layer "B.Cu") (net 23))
 (segment (start 154.315 50.683) (end 153.924 50.292) (width 0.25) (layer "F.Cu") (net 24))
 (segment (start 156.43 100.08) (end 154.156 97.806) (width 0.25) (layer "F.Cu") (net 24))
 (segment (start 154.156 75.203208) (end 154.315 75.044208) (width 0.25) (layer "F.Cu") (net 24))
 (segment (start 154.315 75.044208) (end 154.315 50.683) (width 0.25) (layer "F.Cu") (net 24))
 (segment (start 154.156 97.806) (end 154.156 75.203208) (width 0.25) (layer "F.Cu") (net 24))
 (via (at 153.924 50.292) (size 0.8) (drill 0.4) (layers "F.Cu" "B.Cu") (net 24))
 (segment (start 153.924 50.292) (end 154.076 50.14) (width 0.25) (layer "B.Cu") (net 24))
 (segment (start 154.076 50.14) (end 157.24 50.14) (width 0.25) (layer "B.Cu") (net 24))
 (segment (start 153.772 50.14) (end 153.924 50.292) (width 0.25) (layer "B.Cu") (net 24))
 (segment (start 154.606 96.986) (end 154.606 75.389604) (width 0.25) (layer "F.Cu") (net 25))
 (segment (start 154.765 48.085) (end 154.432 47.752) (width 0.25) (layer "F.Cu") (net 25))
 (segment (start 154.606 75.389604) (end 154.765 75.230604) (width 0.25) (layer "F.Cu") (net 25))
 (segment (start 156.43 98.81) (end 154.606 96.986) (width 0.25) (layer "F.Cu") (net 25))
 (segment (start 154.765 75.230604) (end 154.765 48.085) (width 0.25) (layer "F.Cu") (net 25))
 (via (at 154.432 47.752) (size 0.8) (drill 0.4) (layers "F.Cu" "B.Cu") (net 25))
 (segment (start 154.584 47.6) (end 154.432 47.752) (width 0.25) (layer "B.Cu") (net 25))
 (segment (start 157.24 47.6) (end 154.584 47.6) (width 0.25) (layer "B.Cu") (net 25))
 (segment (start 154.432 47.752) (end 154.28 47.6) (width 0.25) (layer "B.Cu") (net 25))
 (segment (start 155.215 75.417) (end 155.215 45.487) (width 0.25) (layer "F.Cu") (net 26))
 (segment (start 155.056 75.576) (end 155.215 75.417) (width 0.25) (layer "F.Cu") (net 26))
 (segment (start 155.215 45.487) (end 154.94 45.212) (width 0.25) (layer "F.Cu") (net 26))
 (segment (start 155.056 96.166) (end 155.056 75.576) (width 0.25) (layer "F.Cu") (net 26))
 (segment (start 156.43 97.54) (end 155.056 96.166) (width 0.25) (layer "F.Cu") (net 26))
 (via (at 154.94 45.212) (size 0.8) (drill 0.4) (layers "F.Cu" "B.Cu") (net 26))
 (segment (start 155.092 45.06) (end 157.24 45.06) (width 0.25) (layer "B.Cu") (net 26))
 (segment (start 154.94 45.212) (end 155.092 45.06) (width 0.25) (layer "B.Cu") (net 26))
 (segment (start 154.788 45.06) (end 154.94 45.212) (width 0.25) (layer "B.Cu") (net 26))
 (segment (start 155.506 75.851) (end 155.665 75.692) (width 0.25) (layer "F.Cu") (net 27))
 (segment (start 155.665 75.692) (end 155.665 43.143) (width 0.25) (layer "F.Cu") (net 27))
 (segment (start 156.43 96.27) (end 155.506 95.346) (width 0.25) (layer "F.Cu") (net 27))
 (segment (start 155.665 43.143) (end 155.194 42.672) (width 0.25) (layer "F.Cu") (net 27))
 (segment (start 155.506 95.346) (end 155.506 75.851) (width 0.25) (layer "F.Cu") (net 27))
 (via (at 155.194 42.672) (size 0.8) (drill 0.4) (layers "F.Cu" "B.Cu") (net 27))
 (segment (start 155.194 42.672) (end 157.088 42.672) (width 0.25) (layer "B.Cu") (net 27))
 (segment (start 157.088 42.672) (end 157.24 42.52) (width 0.25) (layer "B.Cu") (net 27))
 (segment (start 155.956 94.526) (end 155.956 76.264) (width 0.25) (layer "F.Cu") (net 28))
 (segment (start 155.956 76.264) (end 156.115 76.105) (width 0.25) (layer "F.Cu") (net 28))
 (segment (start 156.115 76.105) (end 156.115 41.105) (width 0.25) (layer "F.Cu") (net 28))
 (segment (start 156.43 95) (end 155.956 94.526) (width 0.25) (layer "F.Cu") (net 28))
 (segment (start 156.115 41.105) (end 157.24 39.98) (width 0.25) (layer "F.Cu") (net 28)))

